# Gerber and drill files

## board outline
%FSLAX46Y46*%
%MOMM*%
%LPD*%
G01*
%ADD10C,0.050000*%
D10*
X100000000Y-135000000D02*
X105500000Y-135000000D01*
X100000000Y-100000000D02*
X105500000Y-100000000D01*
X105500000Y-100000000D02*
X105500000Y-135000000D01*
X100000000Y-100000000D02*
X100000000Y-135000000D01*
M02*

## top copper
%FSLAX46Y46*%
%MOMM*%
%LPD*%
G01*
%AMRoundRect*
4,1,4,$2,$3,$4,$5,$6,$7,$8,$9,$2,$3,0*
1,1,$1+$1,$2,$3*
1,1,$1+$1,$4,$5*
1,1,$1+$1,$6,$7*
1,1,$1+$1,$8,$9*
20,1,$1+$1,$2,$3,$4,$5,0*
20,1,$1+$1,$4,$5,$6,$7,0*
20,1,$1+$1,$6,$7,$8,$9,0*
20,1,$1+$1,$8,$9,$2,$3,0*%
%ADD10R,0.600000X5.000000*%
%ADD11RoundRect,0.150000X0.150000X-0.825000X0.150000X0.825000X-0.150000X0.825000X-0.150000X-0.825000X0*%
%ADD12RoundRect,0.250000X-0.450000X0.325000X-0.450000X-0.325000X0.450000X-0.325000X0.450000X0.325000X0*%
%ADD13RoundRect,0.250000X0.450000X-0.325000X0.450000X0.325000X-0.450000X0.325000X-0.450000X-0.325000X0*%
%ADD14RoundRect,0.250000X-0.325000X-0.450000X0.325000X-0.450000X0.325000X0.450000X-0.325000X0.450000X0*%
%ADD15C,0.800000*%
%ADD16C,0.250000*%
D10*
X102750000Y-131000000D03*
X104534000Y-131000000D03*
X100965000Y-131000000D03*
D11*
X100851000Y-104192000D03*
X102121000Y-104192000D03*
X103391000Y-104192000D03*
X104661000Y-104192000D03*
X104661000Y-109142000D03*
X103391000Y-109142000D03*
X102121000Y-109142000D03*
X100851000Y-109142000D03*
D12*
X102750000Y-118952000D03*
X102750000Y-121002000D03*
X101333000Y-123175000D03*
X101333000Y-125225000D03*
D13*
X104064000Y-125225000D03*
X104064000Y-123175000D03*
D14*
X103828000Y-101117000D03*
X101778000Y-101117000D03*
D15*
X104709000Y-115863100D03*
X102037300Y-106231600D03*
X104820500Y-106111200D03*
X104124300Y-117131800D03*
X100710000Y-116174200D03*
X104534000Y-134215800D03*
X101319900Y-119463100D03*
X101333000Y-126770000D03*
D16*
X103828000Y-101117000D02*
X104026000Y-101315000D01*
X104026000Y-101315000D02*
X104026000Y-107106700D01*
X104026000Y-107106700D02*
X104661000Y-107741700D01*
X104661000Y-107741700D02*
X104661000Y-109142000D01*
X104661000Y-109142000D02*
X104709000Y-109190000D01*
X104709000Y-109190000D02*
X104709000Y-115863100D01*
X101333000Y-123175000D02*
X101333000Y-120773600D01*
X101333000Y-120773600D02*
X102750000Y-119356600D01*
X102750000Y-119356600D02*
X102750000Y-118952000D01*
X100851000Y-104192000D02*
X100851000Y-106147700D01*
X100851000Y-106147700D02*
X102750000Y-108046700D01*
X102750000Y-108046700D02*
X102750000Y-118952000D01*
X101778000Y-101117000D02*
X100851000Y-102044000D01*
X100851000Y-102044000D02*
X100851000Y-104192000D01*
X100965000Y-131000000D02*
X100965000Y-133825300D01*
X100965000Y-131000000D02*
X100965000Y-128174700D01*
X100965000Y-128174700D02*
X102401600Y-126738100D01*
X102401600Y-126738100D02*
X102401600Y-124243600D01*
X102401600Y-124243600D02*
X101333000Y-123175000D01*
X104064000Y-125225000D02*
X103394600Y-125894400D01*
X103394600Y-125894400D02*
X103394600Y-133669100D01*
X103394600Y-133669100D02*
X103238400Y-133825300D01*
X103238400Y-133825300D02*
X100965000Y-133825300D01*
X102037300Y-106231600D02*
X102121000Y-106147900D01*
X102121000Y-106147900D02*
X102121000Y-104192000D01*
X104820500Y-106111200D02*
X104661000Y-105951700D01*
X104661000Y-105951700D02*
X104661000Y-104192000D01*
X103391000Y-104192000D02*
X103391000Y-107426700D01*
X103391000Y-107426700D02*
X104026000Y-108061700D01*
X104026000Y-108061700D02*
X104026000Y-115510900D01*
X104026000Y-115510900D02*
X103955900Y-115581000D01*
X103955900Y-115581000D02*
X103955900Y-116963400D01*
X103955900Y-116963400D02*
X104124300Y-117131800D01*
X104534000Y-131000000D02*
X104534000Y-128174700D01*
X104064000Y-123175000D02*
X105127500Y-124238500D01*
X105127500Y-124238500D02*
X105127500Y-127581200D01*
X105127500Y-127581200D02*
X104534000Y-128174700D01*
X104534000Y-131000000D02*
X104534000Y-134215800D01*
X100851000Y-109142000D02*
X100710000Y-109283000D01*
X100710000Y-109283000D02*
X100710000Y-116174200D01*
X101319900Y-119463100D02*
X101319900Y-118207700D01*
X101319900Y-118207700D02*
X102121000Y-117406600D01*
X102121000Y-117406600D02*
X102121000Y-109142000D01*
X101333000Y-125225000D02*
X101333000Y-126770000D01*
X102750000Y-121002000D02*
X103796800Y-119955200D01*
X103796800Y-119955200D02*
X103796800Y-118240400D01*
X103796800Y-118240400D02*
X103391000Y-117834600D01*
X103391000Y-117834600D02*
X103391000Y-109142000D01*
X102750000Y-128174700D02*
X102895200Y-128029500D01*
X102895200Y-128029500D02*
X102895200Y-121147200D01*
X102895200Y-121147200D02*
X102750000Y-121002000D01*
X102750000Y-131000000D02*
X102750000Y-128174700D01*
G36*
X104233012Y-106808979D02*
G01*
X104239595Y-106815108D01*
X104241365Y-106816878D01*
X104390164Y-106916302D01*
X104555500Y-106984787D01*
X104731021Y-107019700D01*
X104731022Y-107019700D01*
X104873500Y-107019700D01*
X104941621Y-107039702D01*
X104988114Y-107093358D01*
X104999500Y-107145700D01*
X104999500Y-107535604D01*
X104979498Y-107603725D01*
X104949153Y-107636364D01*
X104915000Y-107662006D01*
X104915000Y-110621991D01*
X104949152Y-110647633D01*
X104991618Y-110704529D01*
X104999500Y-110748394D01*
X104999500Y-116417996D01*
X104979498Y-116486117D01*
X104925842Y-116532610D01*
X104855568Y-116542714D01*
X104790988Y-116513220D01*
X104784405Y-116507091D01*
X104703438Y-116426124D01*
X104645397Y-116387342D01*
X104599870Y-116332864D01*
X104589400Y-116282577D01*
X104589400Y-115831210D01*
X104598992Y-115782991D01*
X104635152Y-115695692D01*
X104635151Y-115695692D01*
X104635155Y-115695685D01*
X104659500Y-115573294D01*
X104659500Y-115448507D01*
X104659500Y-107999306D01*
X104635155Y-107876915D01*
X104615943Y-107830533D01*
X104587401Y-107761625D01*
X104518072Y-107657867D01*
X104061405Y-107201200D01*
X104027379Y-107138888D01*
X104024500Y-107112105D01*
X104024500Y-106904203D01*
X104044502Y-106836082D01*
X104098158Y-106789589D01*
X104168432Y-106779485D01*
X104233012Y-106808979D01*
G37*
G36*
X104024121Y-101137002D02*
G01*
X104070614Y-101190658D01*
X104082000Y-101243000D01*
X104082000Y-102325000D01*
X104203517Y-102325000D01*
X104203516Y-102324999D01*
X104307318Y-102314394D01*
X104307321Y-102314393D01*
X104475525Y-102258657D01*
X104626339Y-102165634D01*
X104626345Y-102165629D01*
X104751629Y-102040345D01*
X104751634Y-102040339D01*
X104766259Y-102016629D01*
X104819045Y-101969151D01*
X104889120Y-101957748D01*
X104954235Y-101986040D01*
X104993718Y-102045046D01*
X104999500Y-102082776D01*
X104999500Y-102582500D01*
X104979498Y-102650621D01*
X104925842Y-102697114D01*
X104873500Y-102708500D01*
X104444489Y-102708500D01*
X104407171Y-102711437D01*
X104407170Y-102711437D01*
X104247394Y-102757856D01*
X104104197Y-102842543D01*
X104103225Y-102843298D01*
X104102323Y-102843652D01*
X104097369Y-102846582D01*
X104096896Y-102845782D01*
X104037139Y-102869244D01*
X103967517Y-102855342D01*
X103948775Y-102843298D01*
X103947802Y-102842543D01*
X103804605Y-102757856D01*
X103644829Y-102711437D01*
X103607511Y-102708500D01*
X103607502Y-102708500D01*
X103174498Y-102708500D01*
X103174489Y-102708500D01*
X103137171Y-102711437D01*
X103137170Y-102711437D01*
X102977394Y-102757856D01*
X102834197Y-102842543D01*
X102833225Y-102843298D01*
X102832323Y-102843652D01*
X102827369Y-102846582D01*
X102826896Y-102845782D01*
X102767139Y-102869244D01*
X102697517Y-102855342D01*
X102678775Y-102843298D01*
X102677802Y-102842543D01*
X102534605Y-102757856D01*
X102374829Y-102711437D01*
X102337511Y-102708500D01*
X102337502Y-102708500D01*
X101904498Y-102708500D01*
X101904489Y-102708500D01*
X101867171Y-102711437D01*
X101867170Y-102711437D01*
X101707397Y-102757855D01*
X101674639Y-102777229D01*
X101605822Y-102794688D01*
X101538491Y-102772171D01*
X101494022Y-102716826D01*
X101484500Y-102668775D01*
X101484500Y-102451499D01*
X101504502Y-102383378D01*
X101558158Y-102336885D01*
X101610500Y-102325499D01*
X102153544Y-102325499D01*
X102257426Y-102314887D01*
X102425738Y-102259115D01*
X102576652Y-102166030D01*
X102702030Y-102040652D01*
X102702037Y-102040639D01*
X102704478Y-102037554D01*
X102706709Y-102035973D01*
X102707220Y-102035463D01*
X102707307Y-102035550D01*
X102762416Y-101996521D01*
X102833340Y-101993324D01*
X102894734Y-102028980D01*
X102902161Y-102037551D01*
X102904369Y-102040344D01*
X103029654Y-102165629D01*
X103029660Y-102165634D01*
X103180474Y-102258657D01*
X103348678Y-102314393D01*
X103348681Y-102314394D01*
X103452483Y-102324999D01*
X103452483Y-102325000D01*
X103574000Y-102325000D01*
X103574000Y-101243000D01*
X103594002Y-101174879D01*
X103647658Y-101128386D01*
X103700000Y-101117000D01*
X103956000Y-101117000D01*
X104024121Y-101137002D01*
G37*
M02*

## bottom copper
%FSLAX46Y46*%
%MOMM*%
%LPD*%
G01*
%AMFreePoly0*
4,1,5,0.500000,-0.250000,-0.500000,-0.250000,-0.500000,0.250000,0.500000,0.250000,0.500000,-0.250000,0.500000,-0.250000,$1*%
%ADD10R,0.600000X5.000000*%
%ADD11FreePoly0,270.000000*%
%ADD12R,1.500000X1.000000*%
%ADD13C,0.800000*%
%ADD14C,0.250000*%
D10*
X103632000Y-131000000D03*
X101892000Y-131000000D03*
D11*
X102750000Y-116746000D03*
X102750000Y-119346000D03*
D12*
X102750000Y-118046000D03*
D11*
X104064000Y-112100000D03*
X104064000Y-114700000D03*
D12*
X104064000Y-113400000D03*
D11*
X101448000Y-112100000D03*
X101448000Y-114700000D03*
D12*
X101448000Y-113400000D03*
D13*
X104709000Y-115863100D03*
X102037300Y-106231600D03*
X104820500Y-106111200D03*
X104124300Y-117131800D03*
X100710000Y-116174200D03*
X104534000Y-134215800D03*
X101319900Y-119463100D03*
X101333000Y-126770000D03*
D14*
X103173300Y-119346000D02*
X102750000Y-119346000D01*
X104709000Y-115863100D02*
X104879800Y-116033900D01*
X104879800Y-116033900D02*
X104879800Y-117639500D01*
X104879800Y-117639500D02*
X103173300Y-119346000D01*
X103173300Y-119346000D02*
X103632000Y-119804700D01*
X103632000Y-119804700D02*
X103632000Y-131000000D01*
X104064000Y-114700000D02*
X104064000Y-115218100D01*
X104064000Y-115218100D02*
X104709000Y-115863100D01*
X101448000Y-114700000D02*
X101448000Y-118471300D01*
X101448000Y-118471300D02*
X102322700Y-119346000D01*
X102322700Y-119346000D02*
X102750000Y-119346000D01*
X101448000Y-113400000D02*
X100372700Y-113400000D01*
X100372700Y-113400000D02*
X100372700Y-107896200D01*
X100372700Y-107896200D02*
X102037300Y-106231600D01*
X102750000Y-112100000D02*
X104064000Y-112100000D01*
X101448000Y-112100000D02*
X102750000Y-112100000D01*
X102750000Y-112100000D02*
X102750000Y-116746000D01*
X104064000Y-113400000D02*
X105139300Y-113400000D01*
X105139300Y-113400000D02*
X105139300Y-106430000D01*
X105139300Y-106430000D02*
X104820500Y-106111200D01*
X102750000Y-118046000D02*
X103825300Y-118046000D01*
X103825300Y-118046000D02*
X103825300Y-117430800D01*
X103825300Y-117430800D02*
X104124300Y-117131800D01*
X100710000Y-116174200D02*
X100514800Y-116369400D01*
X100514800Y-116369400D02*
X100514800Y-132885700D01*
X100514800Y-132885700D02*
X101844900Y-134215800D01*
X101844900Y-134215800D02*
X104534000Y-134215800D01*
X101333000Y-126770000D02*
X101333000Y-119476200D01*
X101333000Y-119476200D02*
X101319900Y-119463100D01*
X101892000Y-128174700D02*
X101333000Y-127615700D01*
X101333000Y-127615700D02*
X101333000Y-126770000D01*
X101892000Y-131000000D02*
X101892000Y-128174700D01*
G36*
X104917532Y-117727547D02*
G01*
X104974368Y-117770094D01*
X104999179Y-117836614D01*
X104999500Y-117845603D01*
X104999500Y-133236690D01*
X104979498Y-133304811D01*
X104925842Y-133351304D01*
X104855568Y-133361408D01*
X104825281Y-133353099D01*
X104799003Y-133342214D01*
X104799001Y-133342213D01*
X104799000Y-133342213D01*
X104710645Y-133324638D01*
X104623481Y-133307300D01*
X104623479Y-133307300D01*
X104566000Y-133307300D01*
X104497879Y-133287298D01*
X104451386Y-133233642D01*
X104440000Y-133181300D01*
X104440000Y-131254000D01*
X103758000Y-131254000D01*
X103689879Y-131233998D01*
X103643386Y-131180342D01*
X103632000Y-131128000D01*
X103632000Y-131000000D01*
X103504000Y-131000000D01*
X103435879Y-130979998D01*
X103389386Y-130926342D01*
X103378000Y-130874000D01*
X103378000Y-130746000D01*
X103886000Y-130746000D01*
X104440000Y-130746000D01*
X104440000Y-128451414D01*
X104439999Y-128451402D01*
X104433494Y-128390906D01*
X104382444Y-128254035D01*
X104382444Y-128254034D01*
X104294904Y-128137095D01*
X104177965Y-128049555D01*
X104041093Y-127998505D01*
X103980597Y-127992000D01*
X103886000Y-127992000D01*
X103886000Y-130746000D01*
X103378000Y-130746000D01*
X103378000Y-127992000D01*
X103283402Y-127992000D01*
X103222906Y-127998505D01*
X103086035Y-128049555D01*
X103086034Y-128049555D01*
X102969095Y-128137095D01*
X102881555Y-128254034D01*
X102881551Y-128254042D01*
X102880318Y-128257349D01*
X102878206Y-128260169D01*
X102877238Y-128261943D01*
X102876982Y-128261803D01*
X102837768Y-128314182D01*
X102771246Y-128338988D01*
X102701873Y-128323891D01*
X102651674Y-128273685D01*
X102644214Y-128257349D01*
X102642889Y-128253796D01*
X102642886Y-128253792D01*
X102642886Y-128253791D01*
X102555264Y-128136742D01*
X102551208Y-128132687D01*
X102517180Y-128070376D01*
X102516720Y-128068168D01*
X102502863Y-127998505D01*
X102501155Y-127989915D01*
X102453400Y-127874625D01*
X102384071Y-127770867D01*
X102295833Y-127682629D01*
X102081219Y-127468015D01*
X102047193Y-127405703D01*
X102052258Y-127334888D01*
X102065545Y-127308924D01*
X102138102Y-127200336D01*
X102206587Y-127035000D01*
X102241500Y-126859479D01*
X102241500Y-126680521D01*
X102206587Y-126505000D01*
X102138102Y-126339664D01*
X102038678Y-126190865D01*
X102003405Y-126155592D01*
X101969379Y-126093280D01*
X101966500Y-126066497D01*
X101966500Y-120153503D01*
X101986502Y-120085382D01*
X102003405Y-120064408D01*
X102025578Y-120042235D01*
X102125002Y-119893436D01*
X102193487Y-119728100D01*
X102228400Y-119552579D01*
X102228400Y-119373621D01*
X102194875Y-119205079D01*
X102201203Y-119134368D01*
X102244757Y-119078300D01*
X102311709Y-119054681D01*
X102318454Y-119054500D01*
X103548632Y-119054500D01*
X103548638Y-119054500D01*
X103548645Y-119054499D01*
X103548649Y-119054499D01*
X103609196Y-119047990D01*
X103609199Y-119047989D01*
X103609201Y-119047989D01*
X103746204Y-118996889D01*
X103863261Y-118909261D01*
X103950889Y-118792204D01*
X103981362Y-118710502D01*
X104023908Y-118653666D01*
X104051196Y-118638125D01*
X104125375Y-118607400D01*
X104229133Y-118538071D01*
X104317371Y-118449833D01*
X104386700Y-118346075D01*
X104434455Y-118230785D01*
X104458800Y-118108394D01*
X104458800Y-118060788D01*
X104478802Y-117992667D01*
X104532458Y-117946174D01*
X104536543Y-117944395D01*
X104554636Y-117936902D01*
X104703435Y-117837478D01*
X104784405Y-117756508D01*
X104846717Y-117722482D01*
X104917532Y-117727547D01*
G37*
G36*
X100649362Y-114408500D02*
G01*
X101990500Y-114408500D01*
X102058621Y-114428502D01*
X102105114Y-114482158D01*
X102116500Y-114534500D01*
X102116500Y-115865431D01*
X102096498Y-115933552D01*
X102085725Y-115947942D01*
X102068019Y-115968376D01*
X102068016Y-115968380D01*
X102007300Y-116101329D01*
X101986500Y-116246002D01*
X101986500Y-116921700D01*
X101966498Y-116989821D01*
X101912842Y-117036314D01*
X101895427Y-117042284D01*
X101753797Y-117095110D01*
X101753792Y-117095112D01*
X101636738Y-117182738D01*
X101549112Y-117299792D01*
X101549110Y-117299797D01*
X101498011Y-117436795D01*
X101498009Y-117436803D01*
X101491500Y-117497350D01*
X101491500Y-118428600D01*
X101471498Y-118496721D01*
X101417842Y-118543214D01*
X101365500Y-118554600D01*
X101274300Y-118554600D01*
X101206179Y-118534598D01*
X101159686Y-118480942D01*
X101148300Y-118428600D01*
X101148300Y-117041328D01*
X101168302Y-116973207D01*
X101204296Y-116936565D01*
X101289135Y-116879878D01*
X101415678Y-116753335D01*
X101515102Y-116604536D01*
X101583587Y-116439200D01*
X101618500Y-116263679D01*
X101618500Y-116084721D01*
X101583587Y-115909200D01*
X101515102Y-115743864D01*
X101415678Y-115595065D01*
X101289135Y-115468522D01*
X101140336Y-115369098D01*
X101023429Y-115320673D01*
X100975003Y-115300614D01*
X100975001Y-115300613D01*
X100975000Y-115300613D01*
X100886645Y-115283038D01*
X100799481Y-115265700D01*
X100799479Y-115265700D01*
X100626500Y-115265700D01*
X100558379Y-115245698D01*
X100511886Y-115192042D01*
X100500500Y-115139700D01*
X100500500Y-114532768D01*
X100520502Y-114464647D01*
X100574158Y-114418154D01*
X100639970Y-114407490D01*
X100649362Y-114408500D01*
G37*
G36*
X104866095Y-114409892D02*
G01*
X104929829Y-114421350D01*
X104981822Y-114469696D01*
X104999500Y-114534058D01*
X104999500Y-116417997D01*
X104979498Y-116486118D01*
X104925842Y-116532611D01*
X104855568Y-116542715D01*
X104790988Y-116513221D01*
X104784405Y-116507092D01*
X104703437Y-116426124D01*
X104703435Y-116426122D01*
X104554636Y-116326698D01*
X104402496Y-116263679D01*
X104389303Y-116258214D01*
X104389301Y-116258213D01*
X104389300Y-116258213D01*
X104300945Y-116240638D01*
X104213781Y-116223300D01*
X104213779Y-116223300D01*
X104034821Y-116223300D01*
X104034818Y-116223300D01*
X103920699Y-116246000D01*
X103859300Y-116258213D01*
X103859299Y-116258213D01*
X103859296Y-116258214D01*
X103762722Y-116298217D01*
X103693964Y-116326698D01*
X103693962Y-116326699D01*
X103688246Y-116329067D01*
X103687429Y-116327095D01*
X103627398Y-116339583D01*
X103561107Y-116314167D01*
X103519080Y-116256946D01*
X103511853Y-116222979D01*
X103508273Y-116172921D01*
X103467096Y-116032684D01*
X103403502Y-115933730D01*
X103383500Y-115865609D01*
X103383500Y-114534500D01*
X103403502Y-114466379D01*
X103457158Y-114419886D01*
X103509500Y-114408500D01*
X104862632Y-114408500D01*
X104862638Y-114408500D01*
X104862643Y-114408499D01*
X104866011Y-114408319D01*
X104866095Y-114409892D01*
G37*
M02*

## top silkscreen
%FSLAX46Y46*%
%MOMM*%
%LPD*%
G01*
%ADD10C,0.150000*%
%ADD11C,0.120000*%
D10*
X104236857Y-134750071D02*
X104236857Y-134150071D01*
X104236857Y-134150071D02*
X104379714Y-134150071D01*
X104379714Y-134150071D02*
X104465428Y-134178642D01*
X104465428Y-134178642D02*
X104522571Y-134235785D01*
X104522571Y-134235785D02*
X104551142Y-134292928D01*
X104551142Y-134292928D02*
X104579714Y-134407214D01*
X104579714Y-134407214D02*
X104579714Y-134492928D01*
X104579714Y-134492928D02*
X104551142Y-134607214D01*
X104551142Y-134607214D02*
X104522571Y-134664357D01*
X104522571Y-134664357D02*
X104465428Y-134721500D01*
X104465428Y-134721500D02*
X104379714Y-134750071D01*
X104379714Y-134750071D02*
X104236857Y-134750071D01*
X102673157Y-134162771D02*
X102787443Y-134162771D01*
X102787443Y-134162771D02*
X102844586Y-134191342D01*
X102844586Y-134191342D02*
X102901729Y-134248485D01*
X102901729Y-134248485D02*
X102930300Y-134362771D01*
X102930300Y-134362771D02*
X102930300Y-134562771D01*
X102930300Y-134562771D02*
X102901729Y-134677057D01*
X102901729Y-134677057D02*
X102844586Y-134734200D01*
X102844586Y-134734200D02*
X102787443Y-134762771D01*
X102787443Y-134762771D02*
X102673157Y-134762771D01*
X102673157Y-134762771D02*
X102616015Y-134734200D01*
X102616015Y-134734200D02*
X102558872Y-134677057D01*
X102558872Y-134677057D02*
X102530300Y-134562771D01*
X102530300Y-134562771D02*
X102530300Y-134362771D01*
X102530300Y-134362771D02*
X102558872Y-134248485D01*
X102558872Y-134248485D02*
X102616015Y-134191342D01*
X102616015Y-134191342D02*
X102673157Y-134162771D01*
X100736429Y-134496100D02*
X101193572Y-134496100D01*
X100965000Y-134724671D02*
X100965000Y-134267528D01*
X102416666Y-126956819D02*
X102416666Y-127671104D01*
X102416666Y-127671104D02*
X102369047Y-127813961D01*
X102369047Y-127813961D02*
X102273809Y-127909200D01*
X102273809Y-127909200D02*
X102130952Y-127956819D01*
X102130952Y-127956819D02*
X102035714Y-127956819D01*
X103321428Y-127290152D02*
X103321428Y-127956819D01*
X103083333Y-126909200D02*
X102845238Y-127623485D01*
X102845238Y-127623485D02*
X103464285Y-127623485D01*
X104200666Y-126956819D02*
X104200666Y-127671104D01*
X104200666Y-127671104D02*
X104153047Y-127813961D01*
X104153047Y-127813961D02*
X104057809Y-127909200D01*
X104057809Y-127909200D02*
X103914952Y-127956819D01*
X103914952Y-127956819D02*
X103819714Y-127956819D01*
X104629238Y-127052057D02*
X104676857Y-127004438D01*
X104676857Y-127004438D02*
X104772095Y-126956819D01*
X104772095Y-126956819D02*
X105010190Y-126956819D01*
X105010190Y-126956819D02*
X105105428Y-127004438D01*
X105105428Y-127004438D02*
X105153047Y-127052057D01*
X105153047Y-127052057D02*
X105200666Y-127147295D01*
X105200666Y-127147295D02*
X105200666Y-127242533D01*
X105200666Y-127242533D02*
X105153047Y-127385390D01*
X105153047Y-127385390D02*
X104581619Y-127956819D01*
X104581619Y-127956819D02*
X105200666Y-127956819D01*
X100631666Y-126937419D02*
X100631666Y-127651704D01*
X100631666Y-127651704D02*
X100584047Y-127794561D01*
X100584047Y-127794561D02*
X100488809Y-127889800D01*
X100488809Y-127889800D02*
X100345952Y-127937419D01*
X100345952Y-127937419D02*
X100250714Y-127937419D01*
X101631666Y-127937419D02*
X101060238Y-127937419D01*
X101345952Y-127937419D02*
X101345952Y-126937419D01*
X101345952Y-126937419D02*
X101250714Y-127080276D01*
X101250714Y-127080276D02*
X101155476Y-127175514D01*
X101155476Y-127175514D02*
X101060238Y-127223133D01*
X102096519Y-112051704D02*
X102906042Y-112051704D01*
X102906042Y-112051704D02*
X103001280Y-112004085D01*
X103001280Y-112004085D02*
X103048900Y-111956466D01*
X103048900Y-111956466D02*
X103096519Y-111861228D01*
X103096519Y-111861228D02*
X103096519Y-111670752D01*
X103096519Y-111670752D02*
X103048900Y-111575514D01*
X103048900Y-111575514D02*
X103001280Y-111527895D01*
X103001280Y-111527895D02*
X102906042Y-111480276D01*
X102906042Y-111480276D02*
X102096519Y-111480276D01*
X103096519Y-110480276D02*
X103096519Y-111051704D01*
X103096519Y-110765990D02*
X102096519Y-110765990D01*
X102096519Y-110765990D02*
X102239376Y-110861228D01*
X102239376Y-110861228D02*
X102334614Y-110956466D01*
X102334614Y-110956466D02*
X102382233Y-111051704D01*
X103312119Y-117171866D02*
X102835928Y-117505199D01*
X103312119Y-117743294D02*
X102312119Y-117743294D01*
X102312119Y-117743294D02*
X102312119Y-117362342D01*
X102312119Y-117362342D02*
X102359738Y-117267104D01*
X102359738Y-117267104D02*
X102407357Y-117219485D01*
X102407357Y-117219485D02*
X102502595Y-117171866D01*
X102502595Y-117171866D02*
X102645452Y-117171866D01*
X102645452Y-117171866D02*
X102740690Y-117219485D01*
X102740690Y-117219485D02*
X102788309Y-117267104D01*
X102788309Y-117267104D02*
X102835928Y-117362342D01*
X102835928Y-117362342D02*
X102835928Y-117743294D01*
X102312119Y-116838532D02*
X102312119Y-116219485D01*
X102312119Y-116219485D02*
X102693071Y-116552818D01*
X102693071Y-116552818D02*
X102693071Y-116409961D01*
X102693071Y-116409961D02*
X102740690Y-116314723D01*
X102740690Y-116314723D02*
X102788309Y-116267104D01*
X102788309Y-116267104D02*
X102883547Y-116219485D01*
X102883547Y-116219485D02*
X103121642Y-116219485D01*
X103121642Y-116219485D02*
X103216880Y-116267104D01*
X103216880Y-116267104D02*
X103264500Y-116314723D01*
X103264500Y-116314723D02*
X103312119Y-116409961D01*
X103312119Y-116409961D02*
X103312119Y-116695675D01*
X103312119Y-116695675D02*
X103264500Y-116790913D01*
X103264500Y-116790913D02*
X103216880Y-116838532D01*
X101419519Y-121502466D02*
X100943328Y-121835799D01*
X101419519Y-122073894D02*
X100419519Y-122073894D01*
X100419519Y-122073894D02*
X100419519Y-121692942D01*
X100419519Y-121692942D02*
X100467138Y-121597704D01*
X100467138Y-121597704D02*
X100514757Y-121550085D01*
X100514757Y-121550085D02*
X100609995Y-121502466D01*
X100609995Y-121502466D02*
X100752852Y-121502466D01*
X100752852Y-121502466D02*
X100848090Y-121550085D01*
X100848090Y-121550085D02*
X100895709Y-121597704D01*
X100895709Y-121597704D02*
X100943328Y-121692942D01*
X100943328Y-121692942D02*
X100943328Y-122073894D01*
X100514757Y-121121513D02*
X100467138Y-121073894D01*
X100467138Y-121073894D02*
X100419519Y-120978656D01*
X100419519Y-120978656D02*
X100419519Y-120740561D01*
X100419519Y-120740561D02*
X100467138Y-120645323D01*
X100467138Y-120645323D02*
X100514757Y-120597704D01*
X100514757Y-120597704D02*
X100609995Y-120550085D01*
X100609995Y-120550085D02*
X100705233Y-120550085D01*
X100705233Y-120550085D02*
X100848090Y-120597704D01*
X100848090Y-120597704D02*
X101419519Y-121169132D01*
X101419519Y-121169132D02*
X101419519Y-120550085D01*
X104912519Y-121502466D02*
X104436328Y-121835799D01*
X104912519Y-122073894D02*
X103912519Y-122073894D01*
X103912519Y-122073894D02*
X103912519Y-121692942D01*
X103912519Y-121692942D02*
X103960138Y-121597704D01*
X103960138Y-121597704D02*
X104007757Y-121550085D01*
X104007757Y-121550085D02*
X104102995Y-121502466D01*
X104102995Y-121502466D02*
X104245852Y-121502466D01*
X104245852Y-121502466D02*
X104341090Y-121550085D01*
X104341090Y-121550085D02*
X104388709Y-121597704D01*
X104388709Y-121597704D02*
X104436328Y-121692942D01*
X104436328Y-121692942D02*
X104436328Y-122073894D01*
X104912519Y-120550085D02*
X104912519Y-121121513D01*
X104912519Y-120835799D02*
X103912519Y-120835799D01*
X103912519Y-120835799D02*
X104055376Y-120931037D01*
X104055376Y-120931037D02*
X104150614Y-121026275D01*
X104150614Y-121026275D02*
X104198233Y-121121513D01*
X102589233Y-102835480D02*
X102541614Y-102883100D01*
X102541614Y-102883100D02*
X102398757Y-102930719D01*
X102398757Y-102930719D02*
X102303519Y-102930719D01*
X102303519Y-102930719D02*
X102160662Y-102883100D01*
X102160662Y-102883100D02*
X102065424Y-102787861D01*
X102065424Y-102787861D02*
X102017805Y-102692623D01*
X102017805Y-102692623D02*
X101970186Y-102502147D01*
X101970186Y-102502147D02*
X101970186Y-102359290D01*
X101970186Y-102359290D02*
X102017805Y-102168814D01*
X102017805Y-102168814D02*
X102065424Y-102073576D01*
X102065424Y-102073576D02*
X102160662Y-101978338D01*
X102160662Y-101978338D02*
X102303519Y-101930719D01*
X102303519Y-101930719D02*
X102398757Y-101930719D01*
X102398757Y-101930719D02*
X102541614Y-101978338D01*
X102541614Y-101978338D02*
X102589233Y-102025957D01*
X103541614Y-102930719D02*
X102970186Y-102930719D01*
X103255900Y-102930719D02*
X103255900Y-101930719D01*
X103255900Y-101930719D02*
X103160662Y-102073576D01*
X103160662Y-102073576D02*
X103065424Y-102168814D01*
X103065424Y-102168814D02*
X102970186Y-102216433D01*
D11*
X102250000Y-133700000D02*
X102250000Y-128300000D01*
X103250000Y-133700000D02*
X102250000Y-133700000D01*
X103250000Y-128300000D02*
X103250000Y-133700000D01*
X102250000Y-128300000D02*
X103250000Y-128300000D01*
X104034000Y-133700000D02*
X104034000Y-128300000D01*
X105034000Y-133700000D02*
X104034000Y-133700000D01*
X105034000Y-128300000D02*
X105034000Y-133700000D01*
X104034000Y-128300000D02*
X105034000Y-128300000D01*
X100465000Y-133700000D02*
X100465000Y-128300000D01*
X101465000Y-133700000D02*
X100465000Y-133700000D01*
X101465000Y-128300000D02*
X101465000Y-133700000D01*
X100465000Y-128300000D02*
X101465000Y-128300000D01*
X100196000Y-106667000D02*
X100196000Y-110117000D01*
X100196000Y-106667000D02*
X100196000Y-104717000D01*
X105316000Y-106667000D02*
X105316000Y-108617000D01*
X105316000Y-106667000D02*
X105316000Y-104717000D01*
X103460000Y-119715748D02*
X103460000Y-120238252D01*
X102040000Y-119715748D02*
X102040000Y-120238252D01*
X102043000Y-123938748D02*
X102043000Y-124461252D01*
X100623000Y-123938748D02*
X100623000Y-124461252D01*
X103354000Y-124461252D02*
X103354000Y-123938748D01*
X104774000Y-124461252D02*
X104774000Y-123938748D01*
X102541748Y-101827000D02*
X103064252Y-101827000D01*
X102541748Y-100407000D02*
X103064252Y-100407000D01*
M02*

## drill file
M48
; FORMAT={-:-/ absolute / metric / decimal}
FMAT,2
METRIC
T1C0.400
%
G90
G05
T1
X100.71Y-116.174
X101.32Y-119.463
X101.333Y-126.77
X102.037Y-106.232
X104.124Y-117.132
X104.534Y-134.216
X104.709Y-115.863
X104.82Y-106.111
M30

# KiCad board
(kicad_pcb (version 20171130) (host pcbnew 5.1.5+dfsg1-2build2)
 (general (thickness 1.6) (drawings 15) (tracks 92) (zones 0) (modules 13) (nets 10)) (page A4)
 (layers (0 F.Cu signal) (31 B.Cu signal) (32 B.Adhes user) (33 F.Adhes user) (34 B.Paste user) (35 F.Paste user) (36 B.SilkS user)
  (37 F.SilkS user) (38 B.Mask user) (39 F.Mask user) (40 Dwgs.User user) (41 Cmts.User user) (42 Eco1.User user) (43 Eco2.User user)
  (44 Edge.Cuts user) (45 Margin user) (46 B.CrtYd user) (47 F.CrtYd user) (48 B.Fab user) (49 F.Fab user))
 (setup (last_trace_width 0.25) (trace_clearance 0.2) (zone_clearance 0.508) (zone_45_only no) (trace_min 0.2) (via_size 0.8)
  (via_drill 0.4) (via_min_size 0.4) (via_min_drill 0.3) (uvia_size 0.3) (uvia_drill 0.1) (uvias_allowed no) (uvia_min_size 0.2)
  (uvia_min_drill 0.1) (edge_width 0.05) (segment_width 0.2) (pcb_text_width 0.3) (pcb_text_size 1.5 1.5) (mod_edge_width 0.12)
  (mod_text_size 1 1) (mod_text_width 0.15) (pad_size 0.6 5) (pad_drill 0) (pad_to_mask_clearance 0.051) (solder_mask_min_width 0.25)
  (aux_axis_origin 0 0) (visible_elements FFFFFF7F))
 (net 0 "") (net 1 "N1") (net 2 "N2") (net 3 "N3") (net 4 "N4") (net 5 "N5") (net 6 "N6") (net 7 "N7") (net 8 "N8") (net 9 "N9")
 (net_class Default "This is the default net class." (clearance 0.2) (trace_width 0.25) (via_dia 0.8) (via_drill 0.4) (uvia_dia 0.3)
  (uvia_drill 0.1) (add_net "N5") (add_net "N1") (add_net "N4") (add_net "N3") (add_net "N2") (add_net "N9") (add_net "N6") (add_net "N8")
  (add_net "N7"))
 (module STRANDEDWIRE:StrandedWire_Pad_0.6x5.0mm (layer B.Cu) (at 103.632 131)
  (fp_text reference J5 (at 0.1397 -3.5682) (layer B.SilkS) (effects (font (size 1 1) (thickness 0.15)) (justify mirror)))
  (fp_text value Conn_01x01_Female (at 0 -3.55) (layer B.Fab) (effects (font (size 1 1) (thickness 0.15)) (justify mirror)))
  (pad 1 smd rect (at 0 0) (size 0.6 5) (layers B.Cu B.Mask) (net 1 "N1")))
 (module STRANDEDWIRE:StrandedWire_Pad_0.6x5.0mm (layer F.Cu) (at 102.75 131)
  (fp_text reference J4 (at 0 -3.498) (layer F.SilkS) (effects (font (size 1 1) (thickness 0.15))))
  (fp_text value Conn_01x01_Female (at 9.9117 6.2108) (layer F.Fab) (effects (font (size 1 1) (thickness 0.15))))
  (fp_line (start -0.5 2.7) (end -0.5 -2.7) (layer F.SilkS) (width 0.12))
  (fp_line (start 0.5 2.7) (end -0.5 2.7) (layer F.SilkS) (width 0.12))
  (fp_line (start 0.5 -2.7) (end 0.5 2.7) (layer F.SilkS) (width 0.12))
  (fp_line (start -0.5 -2.7) (end 0.5 -2.7) (layer F.SilkS) (width 0.12))
  (pad 1 smd rect (at 0 0) (size 0.6 5) (layers F.Cu F.Mask) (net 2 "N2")))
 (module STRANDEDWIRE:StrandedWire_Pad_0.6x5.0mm (layer B.Cu) (at 101.892 131)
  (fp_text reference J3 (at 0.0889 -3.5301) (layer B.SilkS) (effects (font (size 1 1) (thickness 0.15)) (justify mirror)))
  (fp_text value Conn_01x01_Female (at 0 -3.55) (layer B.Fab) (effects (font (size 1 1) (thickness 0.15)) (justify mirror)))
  (pad 1 smd rect (at 0 0) (size 0.6 5) (layers B.Cu B.Mask) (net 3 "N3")))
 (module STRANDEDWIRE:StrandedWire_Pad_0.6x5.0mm (layer F.Cu) (at 104.534 131)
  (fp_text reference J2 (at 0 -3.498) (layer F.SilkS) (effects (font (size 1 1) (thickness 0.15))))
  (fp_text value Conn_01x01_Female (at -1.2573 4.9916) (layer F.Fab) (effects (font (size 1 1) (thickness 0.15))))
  (fp_line (start -0.5 2.7) (end -0.5 -2.7) (layer F.SilkS) (width 0.12))
  (fp_line (start 0.5 2.7) (end -0.5 2.7) (layer F.SilkS) (width 0.12))
  (fp_line (start 0.5 -2.7) (end 0.5 2.7) (layer F.SilkS) (width 0.12))
  (fp_line (start -0.5 -2.7) (end 0.5 -2.7) (layer F.SilkS) (width 0.12))
  (pad 1 smd rect (at 0 0) (size 0.6 5) (layers F.Cu F.Mask) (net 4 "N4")))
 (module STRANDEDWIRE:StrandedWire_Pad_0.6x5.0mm (layer F.Cu) (at 100.965 131)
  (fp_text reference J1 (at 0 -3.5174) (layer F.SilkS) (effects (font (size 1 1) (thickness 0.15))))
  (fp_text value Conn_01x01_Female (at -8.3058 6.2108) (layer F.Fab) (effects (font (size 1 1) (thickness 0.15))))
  (fp_line (start -0.5 2.7) (end -0.5 -2.7) (layer F.SilkS) (width 0.12))
  (fp_line (start 0.5 2.7) (end -0.5 2.7) (layer F.SilkS) (width 0.12))
  (fp_line (start 0.5 -2.7) (end 0.5 2.7) (layer F.SilkS) (width 0.12))
  (fp_line (start -0.5 -2.7) (end 0.5 -2.7) (layer F.SilkS) (width 0.12))
  (pad 1 smd rect (at 0 0) (size 0.6 5) (layers F.Cu F.Mask) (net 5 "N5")))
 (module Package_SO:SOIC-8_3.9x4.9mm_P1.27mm (layer F.Cu) (at 102.756 106.667 90)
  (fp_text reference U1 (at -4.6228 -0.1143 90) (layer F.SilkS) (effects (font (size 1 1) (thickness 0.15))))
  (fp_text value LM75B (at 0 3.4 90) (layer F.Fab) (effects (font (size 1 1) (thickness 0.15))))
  (fp_line (start 0 -2.56) (end -3.45 -2.56) (layer F.SilkS) (width 0.12))
  (fp_line (start 0 -2.56) (end 1.95 -2.56) (layer F.SilkS) (width 0.12))
  (fp_line (start 0 2.56) (end -1.95 2.56) (layer F.SilkS) (width 0.12))
  (fp_line (start 0 2.56) (end 1.95 2.56) (layer F.SilkS) (width 0.12))
  (pad 8 smd roundrect (at 2.475 -1.905 90) (size 1.95 0.6) (layers F.Cu F.Paste F.Mask) (roundrect_rratio 0.25) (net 5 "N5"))
  (pad 7 smd roundrect (at 2.475 -0.635 90) (size 1.95 0.6) (layers F.Cu F.Paste F.Mask) (roundrect_rratio 0.25) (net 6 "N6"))
  (pad 6 smd roundrect (at 2.475 0.635 90) (size 1.95 0.6) (layers F.Cu F.Paste F.Mask) (roundrect_rratio 0.25) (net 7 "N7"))
  (pad 5 smd roundrect (at 2.475 1.905 90) (size 1.95 0.6) (layers F.Cu F.Paste F.Mask) (roundrect_rratio 0.25) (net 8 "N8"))
  (pad 4 smd roundrect (at -2.475 1.905 90) (size 1.95 0.6) (layers F.Cu F.Paste F.Mask) (roundrect_rratio 0.25) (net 1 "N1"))
  (pad 3 smd roundrect (at -2.475 0.635 90) (size 1.95 0.6) (layers F.Cu F.Paste F.Mask) (roundrect_rratio 0.25) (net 2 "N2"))
  (pad 2 smd roundrect (at -2.475 -0.635 90) (size 1.95 0.6) (layers F.Cu F.Paste F.Mask) (roundrect_rratio 0.25) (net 3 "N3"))
  (pad 1 smd roundrect (at -2.475 -1.905 90) (size 1.95 0.6) (layers F.Cu F.Paste F.Mask) (roundrect_rratio 0.25) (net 4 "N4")))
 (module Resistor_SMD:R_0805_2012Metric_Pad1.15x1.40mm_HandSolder (layer F.Cu) (at 102.75 119.977 270)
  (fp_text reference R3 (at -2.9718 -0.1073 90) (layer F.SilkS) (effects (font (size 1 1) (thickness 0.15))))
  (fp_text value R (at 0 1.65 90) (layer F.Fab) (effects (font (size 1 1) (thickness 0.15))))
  (fp_line (start -0.261252 -0.71) (end 0.261252 -0.71) (layer F.SilkS) (width 0.12))
  (fp_line (start -0.261252 0.71) (end 0.261252 0.71) (layer F.SilkS) (width 0.12))
  (pad 1 smd roundrect (at -1.025 0 270) (size 1.15 1.4) (layers F.Cu F.Paste F.Mask) (roundrect_rratio 0.217391) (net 5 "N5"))
  (pad 2 smd roundrect (at 1.025 0 270) (size 1.15 1.4) (layers F.Cu F.Paste F.Mask) (roundrect_rratio 0.217391) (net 2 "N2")))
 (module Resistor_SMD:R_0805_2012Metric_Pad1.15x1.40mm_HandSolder (layer F.Cu) (at 101.333 124.2 270)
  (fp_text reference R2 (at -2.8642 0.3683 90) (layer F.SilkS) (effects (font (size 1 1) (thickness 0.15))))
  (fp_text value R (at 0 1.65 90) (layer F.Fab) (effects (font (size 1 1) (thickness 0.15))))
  (fp_line (start -0.261252 -0.71) (end 0.261252 -0.71) (layer F.SilkS) (width 0.12))
  (fp_line (start -0.261252 0.71) (end 0.261252 0.71) (layer F.SilkS) (width 0.12))
  (pad 1 smd roundrect (at -1.025 0 270) (size 1.15 1.4) (layers F.Cu F.Paste F.Mask) (roundrect_rratio 0.217391) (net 5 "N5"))
  (pad 2 smd roundrect (at 1.025 0 270) (size 1.15 1.4) (layers F.Cu F.Paste F.Mask) (roundrect_rratio 0.217391) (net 3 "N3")))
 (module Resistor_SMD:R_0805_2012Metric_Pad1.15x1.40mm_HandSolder (layer F.Cu) (at 104.064 124.2 90)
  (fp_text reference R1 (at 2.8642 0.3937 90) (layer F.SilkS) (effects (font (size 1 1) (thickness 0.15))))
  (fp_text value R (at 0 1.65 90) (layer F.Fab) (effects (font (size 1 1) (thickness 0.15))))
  (fp_line (start -0.261252 -0.71) (end 0.261252 -0.71) (layer F.SilkS) (width 0.12))
  (fp_line (start -0.261252 0.71) (end 0.261252 0.71) (layer F.SilkS) (width 0.12))
  (pad 1 smd roundrect (at -1.025 0 90) (size 1.15 1.4) (layers F.Cu F.Paste F.Mask) (roundrect_rratio 0.217391) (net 5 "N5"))
  (pad 2 smd roundrect (at 1.025 0 90) (size 1.15 1.4) (layers F.Cu F.Paste F.Mask) (roundrect_rratio 0.217391) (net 4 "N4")))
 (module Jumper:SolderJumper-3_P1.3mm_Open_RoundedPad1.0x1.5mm (layer B.Cu) (at 102.75 118.046 270)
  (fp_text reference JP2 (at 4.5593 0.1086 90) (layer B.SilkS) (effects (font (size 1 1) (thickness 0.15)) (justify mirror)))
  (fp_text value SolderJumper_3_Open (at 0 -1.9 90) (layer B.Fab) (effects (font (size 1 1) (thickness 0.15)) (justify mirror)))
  (pad 1 smd custom (at -1.3 0 270) (size 1 0.5) (layers B.Cu B.Mask) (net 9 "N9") (zone_connect 2)
   (options (clearance outline) (anchor rect)) (primitives))
  (pad 3 smd custom (at 1.3 0 270) (size 1 0.5) (layers B.Cu B.Mask) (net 1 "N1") (zone_connect 2)
   (options (clearance outline) (anchor rect)) (primitives))
  (pad 2 smd rect (at 0 0 270) (size 1 1.5) (layers B.Cu B.Mask) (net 7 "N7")))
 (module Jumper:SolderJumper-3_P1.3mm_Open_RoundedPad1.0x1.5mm (layer B.Cu) (at 104.064 113.4 270)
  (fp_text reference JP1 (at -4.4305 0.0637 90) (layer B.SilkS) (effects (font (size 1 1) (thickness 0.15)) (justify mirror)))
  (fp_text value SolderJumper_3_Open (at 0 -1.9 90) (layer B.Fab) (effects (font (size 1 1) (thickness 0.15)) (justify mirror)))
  (pad 1 smd custom (at -1.3 0 270) (size 1 0.5) (layers B.Cu B.Mask) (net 9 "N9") (zone_connect 2)
   (options (clearance outline) (anchor rect)) (primitives))
  (pad 3 smd custom (at 1.3 0 270) (size 1 0.5) (layers B.Cu B.Mask) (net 1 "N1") (zone_connect 2)
   (options (clearance outline) (anchor rect)) (primitives))
  (pad 2 smd rect (at 0 0 270) (size 1 1.5) (layers B.Cu B.Mask) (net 8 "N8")))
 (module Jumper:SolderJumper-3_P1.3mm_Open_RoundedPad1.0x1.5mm (layer B.Cu) (at 101.448 113.4 270)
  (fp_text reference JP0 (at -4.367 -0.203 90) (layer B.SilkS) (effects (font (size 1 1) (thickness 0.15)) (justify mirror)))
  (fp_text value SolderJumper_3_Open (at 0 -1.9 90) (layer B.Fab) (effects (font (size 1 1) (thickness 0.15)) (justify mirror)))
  (pad 1 smd custom (at -1.3 0 270) (size 1 0.5) (layers B.Cu B.Mask) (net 9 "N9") (zone_connect 2)
   (options (clearance outline) (anchor rect)) (primitives))
  (pad 3 smd custom (at 1.3 0 270) (size 1 0.5) (layers B.Cu B.Mask) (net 1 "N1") (zone_connect 2)
   (options (clearance outline) (anchor rect)) (primitives))
  (pad 2 smd rect (at 0 0 270) (size 1 1.5) (layers B.Cu B.Mask) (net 6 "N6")))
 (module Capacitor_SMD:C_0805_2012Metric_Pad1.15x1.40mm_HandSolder (layer F.Cu) (at 102.803 101.117)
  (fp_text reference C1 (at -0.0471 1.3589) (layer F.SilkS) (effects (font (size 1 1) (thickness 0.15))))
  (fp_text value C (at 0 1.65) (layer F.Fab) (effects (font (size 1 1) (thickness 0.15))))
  (fp_line (start -0.261252 0.71) (end 0.261252 0.71) (layer F.SilkS) (width 0.12))
  (fp_line (start -0.261252 -0.71) (end 0.261252 -0.71) (layer F.SilkS) (width 0.12))
  (pad 2 smd roundrect (at 1.025 0) (size 1.15 1.4) (layers F.Cu F.Paste F.Mask) (roundrect_rratio 0.217391) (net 1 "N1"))
  (pad 1 smd roundrect (at -1.025 0) (size 1.15 1.4) (layers F.Cu F.Paste F.Mask) (roundrect_rratio 0.217391) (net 5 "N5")))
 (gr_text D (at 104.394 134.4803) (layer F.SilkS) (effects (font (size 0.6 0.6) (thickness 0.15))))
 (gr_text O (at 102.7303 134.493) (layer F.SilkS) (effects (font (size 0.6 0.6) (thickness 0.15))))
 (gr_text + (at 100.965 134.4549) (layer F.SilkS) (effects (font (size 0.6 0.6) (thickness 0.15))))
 (gr_line (start 100 135) (end 105.5 135) (layer Edge.Cuts) (width 0.05))
 (gr_line (start 100 100) (end 105.5 100) (layer Edge.Cuts) (width 0.05))
 (gr_line (start 105.5 100) (end 105.5 135) (layer Edge.Cuts) (width 0.05))
 (gr_line (start 100 100) (end 100 135) (layer Edge.Cuts) (width 0.05))
 (segment (start 103.828 101.117) (end 104.026 101.315) (width 0.25) (layer F.Cu) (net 1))
 (segment (start 104.026 101.315) (end 104.026 107.1067) (width 0.25) (layer F.Cu) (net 1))
 (segment (start 104.026 107.1067) (end 104.661 107.7417) (width 0.25) (layer F.Cu) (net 1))
 (segment (start 104.661 107.7417) (end 104.661 109.142) (width 0.25) (layer F.Cu) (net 1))
 (segment (start 103.1733 119.346) (end 102.75 119.346) (width 0.25) (layer B.Cu) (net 1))
 (segment (start 104.709 115.8631) (end 104.8798 116.0339) (width 0.25) (layer B.Cu) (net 1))
 (segment (start 104.8798 116.0339) (end 104.8798 117.6395) (width 0.25) (layer B.Cu) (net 1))
 (segment (start 104.8798 117.6395) (end 103.1733 119.346) (width 0.25) (layer B.Cu) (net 1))
 (segment (start 103.1733 119.346) (end 103.632 119.8047) (width 0.25) (layer B.Cu) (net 1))
 (segment (start 103.632 119.8047) (end 103.632 131) (width 0.25) (layer B.Cu) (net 1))
 (segment (start 104.064 114.7) (end 104.064 115.2181) (width 0.25) (layer B.Cu) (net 1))
 (segment (start 104.064 115.2181) (end 104.709 115.8631) (width 0.25) (layer B.Cu) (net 1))
 (segment (start 104.661 109.142) (end 104.709 109.19) (width 0.25) (layer F.Cu) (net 1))
 (segment (start 104.709 109.19) (end 104.709 115.8631) (width 0.25) (layer F.Cu) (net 1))
 (segment (start 101.448 114.7) (end 101.448 118.4713) (width 0.25) (layer B.Cu) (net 1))
 (segment (start 101.448 118.4713) (end 102.3227 119.346) (width 0.25) (layer B.Cu) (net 1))
 (segment (start 102.3227 119.346) (end 102.75 119.346) (width 0.25) (layer B.Cu) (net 1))
 (via (at 104.709 115.8631) (size 0.8) (layers F.Cu B.Cu) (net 1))
 (segment (start 101.333 123.175) (end 101.333 120.7736) (width 0.25) (layer F.Cu) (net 5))
 (segment (start 101.333 120.7736) (end 102.75 119.3566) (width 0.25) (layer F.Cu) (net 5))
 (segment (start 102.75 119.3566) (end 102.75 118.952) (width 0.25) (layer F.Cu) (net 5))
 (segment (start 100.851 104.192) (end 100.851 106.1477) (width 0.25) (layer F.Cu) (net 5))
 (segment (start 100.851 106.1477) (end 102.75 108.0467) (width 0.25) (layer F.Cu) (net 5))
 (segment (start 102.75 108.0467) (end 102.75 118.952) (width 0.25) (layer F.Cu) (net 5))
 (segment (start 101.778 101.117) (end 100.851 102.044) (width 0.25) (layer F.Cu) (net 5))
 (segment (start 100.851 102.044) (end 100.851 104.192) (width 0.25) (layer F.Cu) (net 5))
 (segment (start 100.965 131) (end 100.965 133.8253) (width 0.25) (layer F.Cu) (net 5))
 (segment (start 100.965 131) (end 100.965 128.1747) (width 0.25) (layer F.Cu) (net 5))
 (segment (start 100.965 128.1747) (end 102.4016 126.7381) (width 0.25) (layer F.Cu) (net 5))
 (segment (start 102.4016 126.7381) (end 102.4016 124.2436) (width 0.25) (layer F.Cu) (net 5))
 (segment (start 102.4016 124.2436) (end 101.333 123.175) (width 0.25) (layer F.Cu) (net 5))
 (segment (start 104.064 125.225) (end 103.3946 125.8944) (width 0.25) (layer F.Cu) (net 5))
 (segment (start 103.3946 125.8944) (end 103.3946 133.6691) (width 0.25) (layer F.Cu) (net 5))
 (segment (start 103.3946 133.6691) (end 103.2384 133.8253) (width 0.25) (layer F.Cu) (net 5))
 (segment (start 103.2384 133.8253) (end 100.965 133.8253) (width 0.25) (layer F.Cu) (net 5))
 (segment (start 101.448 113.4) (end 100.3727 113.4) (width 0.25) (layer B.Cu) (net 6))
 (segment (start 102.0373 106.2316) (end 102.121 106.1479) (width 0.25) (layer F.Cu) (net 6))
 (segment (start 102.121 106.1479) (end 102.121 104.192) (width 0.25) (layer F.Cu) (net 6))
 (segment (start 100.3727 113.4) (end 100.3727 107.8962) (width 0.25) (layer B.Cu) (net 6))
 (segment (start 100.3727 107.8962) (end 102.0373 106.2316) (width 0.25) (layer B.Cu) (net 6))
 (via (at 102.0373 106.2316) (size 0.8) (layers F.Cu B.Cu) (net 6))
 (segment (start 102.75 112.1) (end 104.064 112.1) (width 0.25) (layer B.Cu) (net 9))
 (segment (start 101.448 112.1) (end 102.75 112.1) (width 0.25) (layer B.Cu) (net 9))
 (segment (start 102.75 112.1) (end 102.75 116.746) (width 0.25) (layer B.Cu) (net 9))
 (segment (start 104.064 113.4) (end 105.1393 113.4) (width 0.25) (layer B.Cu) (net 8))
 (segment (start 104.8205 106.1112) (end 104.661 105.9517) (width 0.25) (layer F.Cu) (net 8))
 (segment (start 104.661 105.9517) (end 104.661 104.192) (width 0.25) (layer F.Cu) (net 8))
 (segment (start 105.1393 113.4) (end 105.1393 106.43) (width 0.25) (layer B.Cu) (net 8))
 (segment (start 105.1393 106.43) (end 104.8205 106.1112) (width 0.25) (layer B.Cu) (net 8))
 (via (at 104.8205 106.1112) (size 0.8) (layers F.Cu B.Cu) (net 8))
 (segment (start 103.391 104.192) (end 103.391 107.4267) (width 0.25) (layer F.Cu) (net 7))
 (segment (start 103.391 107.4267) (end 104.026 108.0617) (width 0.25) (layer F.Cu) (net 7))
 (segment (start 104.026 108.0617) (end 104.026 115.5109) (width 0.25) (layer F.Cu) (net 7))
 (segment (start 104.026 115.5109) (end 103.9559 115.581) (width 0.25) (layer F.Cu) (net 7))
 (segment (start 103.9559 115.581) (end 103.9559 116.9634) (width 0.25) (layer F.Cu) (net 7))
 (segment (start 103.9559 116.9634) (end 104.1243 117.1318) (width 0.25) (layer F.Cu) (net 7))
 (segment (start 102.75 118.046) (end 103.8253 118.046) (width 0.25) (layer B.Cu) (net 7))
 (segment (start 103.8253 118.046) (end 103.8253 117.4308) (width 0.25) (layer B.Cu) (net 7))
 (segment (start 103.8253 117.4308) (end 104.1243 117.1318) (width 0.25) (layer B.Cu) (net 7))
 (via (at 104.1243 117.1318) (size 0.8) (layers F.Cu B.Cu) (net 7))
 (segment (start 104.534 131) (end 104.534 128.1747) (width 0.25) (layer F.Cu) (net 4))
 (segment (start 104.064 123.175) (end 105.1275 124.2385) (width 0.25) (layer F.Cu) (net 4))
 (segment (start 105.1275 124.2385) (end 105.1275 127.5812) (width 0.25) (layer F.Cu) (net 4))
 (segment (start 105.1275 127.5812) (end 104.534 128.1747) (width 0.25) (layer F.Cu) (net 4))
 (segment (start 104.534 131) (end 104.534 134.2158) (width 0.25) (layer F.Cu) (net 4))
 (segment (start 100.71 116.1742) (end 100.5148 116.3694) (width 0.25) (layer B.Cu) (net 4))
 (segment (start 100.5148 116.3694) (end 100.5148 132.8857) (width 0.25) (layer B.Cu) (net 4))
 (segment (start 100.5148 132.8857) (end 101.8449 134.2158) (width 0.25) (layer B.Cu) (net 4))
 (segment (start 101.8449 134.2158) (end 104.534 134.2158) (width 0.25) (layer B.Cu) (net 4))
 (segment (start 100.851 109.142) (end 100.71 109.283) (width 0.25) (layer F.Cu) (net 4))
 (segment (start 100.71 109.283) (end 100.71 116.1742) (width 0.25) (layer F.Cu) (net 4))
 (via (at 100.71 116.1742) (size 0.8) (layers F.Cu B.Cu) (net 4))
 (via (at 104.534 134.2158) (size 0.8) (layers F.Cu B.Cu) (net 4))
 (segment (start 101.3199 119.4631) (end 101.3199 118.2077) (width 0.25) (layer F.Cu) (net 3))
 (segment (start 101.3199 118.2077) (end 102.121 117.4066) (width 0.25) (layer F.Cu) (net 3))
 (segment (start 102.121 117.4066) (end 102.121 109.142) (width 0.25) (layer F.Cu) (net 3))
 (segment (start 101.333 126.77) (end 101.333 119.4762) (width 0.25) (layer B.Cu) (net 3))
 (segment (start 101.333 119.4762) (end 101.3199 119.4631) (width 0.25) (layer B.Cu) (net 3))
 (segment (start 101.892 128.1747) (end 101.333 127.6157) (width 0.25) (layer B.Cu) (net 3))
 (segment (start 101.333 127.6157) (end 101.333 126.77) (width 0.25) (layer B.Cu) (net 3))
 (segment (start 101.333 125.225) (end 101.333 126.77) (width 0.25) (layer F.Cu) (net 3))
 (segment (start 101.892 131) (end 101.892 128.1747) (width 0.25) (layer B.Cu) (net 3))
 (via (at 101.3199 119.4631) (size 0.8) (layers F.Cu B.Cu) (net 3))
 (via (at 101.333 126.77) (size 0.8) (layers F.Cu B.Cu) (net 3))
 (segment (start 102.75 121.002) (end 103.7968 119.9552) (width 0.25) (layer F.Cu) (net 2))
 (segment (start 103.7968 119.9552) (end 103.7968 118.2404) (width 0.25) (layer F.Cu) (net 2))
 (segment (start 103.7968 118.2404) (end 103.391 117.8346) (width 0.25) (layer F.Cu) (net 2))
 (segment (start 103.391 117.8346) (end 103.391 109.142) (width 0.25) (layer F.Cu) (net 2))
 (segment (start 102.75 128.1747) (end 102.8952 128.0295) (width 0.25) (layer F.Cu) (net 2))
 (segment (start 102.8952 128.0295) (end 102.8952 121.1472) (width 0.25) (layer F.Cu) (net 2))
 (segment (start 102.8952 121.1472) (end 102.75 121.002) (width 0.25) (layer F.Cu) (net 2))
 (segment (start 102.75 131) (end 102.75 128.1747) (width 0.25) (layer F.Cu) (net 2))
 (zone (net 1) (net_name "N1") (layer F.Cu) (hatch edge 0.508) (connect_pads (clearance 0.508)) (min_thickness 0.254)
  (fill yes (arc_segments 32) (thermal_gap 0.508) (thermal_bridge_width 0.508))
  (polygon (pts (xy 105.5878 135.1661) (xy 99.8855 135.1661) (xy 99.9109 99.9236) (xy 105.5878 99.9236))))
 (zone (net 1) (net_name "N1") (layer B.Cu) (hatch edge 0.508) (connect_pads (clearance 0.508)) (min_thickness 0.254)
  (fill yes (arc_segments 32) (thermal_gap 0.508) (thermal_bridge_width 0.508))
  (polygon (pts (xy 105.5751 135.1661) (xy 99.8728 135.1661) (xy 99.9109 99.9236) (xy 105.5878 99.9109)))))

